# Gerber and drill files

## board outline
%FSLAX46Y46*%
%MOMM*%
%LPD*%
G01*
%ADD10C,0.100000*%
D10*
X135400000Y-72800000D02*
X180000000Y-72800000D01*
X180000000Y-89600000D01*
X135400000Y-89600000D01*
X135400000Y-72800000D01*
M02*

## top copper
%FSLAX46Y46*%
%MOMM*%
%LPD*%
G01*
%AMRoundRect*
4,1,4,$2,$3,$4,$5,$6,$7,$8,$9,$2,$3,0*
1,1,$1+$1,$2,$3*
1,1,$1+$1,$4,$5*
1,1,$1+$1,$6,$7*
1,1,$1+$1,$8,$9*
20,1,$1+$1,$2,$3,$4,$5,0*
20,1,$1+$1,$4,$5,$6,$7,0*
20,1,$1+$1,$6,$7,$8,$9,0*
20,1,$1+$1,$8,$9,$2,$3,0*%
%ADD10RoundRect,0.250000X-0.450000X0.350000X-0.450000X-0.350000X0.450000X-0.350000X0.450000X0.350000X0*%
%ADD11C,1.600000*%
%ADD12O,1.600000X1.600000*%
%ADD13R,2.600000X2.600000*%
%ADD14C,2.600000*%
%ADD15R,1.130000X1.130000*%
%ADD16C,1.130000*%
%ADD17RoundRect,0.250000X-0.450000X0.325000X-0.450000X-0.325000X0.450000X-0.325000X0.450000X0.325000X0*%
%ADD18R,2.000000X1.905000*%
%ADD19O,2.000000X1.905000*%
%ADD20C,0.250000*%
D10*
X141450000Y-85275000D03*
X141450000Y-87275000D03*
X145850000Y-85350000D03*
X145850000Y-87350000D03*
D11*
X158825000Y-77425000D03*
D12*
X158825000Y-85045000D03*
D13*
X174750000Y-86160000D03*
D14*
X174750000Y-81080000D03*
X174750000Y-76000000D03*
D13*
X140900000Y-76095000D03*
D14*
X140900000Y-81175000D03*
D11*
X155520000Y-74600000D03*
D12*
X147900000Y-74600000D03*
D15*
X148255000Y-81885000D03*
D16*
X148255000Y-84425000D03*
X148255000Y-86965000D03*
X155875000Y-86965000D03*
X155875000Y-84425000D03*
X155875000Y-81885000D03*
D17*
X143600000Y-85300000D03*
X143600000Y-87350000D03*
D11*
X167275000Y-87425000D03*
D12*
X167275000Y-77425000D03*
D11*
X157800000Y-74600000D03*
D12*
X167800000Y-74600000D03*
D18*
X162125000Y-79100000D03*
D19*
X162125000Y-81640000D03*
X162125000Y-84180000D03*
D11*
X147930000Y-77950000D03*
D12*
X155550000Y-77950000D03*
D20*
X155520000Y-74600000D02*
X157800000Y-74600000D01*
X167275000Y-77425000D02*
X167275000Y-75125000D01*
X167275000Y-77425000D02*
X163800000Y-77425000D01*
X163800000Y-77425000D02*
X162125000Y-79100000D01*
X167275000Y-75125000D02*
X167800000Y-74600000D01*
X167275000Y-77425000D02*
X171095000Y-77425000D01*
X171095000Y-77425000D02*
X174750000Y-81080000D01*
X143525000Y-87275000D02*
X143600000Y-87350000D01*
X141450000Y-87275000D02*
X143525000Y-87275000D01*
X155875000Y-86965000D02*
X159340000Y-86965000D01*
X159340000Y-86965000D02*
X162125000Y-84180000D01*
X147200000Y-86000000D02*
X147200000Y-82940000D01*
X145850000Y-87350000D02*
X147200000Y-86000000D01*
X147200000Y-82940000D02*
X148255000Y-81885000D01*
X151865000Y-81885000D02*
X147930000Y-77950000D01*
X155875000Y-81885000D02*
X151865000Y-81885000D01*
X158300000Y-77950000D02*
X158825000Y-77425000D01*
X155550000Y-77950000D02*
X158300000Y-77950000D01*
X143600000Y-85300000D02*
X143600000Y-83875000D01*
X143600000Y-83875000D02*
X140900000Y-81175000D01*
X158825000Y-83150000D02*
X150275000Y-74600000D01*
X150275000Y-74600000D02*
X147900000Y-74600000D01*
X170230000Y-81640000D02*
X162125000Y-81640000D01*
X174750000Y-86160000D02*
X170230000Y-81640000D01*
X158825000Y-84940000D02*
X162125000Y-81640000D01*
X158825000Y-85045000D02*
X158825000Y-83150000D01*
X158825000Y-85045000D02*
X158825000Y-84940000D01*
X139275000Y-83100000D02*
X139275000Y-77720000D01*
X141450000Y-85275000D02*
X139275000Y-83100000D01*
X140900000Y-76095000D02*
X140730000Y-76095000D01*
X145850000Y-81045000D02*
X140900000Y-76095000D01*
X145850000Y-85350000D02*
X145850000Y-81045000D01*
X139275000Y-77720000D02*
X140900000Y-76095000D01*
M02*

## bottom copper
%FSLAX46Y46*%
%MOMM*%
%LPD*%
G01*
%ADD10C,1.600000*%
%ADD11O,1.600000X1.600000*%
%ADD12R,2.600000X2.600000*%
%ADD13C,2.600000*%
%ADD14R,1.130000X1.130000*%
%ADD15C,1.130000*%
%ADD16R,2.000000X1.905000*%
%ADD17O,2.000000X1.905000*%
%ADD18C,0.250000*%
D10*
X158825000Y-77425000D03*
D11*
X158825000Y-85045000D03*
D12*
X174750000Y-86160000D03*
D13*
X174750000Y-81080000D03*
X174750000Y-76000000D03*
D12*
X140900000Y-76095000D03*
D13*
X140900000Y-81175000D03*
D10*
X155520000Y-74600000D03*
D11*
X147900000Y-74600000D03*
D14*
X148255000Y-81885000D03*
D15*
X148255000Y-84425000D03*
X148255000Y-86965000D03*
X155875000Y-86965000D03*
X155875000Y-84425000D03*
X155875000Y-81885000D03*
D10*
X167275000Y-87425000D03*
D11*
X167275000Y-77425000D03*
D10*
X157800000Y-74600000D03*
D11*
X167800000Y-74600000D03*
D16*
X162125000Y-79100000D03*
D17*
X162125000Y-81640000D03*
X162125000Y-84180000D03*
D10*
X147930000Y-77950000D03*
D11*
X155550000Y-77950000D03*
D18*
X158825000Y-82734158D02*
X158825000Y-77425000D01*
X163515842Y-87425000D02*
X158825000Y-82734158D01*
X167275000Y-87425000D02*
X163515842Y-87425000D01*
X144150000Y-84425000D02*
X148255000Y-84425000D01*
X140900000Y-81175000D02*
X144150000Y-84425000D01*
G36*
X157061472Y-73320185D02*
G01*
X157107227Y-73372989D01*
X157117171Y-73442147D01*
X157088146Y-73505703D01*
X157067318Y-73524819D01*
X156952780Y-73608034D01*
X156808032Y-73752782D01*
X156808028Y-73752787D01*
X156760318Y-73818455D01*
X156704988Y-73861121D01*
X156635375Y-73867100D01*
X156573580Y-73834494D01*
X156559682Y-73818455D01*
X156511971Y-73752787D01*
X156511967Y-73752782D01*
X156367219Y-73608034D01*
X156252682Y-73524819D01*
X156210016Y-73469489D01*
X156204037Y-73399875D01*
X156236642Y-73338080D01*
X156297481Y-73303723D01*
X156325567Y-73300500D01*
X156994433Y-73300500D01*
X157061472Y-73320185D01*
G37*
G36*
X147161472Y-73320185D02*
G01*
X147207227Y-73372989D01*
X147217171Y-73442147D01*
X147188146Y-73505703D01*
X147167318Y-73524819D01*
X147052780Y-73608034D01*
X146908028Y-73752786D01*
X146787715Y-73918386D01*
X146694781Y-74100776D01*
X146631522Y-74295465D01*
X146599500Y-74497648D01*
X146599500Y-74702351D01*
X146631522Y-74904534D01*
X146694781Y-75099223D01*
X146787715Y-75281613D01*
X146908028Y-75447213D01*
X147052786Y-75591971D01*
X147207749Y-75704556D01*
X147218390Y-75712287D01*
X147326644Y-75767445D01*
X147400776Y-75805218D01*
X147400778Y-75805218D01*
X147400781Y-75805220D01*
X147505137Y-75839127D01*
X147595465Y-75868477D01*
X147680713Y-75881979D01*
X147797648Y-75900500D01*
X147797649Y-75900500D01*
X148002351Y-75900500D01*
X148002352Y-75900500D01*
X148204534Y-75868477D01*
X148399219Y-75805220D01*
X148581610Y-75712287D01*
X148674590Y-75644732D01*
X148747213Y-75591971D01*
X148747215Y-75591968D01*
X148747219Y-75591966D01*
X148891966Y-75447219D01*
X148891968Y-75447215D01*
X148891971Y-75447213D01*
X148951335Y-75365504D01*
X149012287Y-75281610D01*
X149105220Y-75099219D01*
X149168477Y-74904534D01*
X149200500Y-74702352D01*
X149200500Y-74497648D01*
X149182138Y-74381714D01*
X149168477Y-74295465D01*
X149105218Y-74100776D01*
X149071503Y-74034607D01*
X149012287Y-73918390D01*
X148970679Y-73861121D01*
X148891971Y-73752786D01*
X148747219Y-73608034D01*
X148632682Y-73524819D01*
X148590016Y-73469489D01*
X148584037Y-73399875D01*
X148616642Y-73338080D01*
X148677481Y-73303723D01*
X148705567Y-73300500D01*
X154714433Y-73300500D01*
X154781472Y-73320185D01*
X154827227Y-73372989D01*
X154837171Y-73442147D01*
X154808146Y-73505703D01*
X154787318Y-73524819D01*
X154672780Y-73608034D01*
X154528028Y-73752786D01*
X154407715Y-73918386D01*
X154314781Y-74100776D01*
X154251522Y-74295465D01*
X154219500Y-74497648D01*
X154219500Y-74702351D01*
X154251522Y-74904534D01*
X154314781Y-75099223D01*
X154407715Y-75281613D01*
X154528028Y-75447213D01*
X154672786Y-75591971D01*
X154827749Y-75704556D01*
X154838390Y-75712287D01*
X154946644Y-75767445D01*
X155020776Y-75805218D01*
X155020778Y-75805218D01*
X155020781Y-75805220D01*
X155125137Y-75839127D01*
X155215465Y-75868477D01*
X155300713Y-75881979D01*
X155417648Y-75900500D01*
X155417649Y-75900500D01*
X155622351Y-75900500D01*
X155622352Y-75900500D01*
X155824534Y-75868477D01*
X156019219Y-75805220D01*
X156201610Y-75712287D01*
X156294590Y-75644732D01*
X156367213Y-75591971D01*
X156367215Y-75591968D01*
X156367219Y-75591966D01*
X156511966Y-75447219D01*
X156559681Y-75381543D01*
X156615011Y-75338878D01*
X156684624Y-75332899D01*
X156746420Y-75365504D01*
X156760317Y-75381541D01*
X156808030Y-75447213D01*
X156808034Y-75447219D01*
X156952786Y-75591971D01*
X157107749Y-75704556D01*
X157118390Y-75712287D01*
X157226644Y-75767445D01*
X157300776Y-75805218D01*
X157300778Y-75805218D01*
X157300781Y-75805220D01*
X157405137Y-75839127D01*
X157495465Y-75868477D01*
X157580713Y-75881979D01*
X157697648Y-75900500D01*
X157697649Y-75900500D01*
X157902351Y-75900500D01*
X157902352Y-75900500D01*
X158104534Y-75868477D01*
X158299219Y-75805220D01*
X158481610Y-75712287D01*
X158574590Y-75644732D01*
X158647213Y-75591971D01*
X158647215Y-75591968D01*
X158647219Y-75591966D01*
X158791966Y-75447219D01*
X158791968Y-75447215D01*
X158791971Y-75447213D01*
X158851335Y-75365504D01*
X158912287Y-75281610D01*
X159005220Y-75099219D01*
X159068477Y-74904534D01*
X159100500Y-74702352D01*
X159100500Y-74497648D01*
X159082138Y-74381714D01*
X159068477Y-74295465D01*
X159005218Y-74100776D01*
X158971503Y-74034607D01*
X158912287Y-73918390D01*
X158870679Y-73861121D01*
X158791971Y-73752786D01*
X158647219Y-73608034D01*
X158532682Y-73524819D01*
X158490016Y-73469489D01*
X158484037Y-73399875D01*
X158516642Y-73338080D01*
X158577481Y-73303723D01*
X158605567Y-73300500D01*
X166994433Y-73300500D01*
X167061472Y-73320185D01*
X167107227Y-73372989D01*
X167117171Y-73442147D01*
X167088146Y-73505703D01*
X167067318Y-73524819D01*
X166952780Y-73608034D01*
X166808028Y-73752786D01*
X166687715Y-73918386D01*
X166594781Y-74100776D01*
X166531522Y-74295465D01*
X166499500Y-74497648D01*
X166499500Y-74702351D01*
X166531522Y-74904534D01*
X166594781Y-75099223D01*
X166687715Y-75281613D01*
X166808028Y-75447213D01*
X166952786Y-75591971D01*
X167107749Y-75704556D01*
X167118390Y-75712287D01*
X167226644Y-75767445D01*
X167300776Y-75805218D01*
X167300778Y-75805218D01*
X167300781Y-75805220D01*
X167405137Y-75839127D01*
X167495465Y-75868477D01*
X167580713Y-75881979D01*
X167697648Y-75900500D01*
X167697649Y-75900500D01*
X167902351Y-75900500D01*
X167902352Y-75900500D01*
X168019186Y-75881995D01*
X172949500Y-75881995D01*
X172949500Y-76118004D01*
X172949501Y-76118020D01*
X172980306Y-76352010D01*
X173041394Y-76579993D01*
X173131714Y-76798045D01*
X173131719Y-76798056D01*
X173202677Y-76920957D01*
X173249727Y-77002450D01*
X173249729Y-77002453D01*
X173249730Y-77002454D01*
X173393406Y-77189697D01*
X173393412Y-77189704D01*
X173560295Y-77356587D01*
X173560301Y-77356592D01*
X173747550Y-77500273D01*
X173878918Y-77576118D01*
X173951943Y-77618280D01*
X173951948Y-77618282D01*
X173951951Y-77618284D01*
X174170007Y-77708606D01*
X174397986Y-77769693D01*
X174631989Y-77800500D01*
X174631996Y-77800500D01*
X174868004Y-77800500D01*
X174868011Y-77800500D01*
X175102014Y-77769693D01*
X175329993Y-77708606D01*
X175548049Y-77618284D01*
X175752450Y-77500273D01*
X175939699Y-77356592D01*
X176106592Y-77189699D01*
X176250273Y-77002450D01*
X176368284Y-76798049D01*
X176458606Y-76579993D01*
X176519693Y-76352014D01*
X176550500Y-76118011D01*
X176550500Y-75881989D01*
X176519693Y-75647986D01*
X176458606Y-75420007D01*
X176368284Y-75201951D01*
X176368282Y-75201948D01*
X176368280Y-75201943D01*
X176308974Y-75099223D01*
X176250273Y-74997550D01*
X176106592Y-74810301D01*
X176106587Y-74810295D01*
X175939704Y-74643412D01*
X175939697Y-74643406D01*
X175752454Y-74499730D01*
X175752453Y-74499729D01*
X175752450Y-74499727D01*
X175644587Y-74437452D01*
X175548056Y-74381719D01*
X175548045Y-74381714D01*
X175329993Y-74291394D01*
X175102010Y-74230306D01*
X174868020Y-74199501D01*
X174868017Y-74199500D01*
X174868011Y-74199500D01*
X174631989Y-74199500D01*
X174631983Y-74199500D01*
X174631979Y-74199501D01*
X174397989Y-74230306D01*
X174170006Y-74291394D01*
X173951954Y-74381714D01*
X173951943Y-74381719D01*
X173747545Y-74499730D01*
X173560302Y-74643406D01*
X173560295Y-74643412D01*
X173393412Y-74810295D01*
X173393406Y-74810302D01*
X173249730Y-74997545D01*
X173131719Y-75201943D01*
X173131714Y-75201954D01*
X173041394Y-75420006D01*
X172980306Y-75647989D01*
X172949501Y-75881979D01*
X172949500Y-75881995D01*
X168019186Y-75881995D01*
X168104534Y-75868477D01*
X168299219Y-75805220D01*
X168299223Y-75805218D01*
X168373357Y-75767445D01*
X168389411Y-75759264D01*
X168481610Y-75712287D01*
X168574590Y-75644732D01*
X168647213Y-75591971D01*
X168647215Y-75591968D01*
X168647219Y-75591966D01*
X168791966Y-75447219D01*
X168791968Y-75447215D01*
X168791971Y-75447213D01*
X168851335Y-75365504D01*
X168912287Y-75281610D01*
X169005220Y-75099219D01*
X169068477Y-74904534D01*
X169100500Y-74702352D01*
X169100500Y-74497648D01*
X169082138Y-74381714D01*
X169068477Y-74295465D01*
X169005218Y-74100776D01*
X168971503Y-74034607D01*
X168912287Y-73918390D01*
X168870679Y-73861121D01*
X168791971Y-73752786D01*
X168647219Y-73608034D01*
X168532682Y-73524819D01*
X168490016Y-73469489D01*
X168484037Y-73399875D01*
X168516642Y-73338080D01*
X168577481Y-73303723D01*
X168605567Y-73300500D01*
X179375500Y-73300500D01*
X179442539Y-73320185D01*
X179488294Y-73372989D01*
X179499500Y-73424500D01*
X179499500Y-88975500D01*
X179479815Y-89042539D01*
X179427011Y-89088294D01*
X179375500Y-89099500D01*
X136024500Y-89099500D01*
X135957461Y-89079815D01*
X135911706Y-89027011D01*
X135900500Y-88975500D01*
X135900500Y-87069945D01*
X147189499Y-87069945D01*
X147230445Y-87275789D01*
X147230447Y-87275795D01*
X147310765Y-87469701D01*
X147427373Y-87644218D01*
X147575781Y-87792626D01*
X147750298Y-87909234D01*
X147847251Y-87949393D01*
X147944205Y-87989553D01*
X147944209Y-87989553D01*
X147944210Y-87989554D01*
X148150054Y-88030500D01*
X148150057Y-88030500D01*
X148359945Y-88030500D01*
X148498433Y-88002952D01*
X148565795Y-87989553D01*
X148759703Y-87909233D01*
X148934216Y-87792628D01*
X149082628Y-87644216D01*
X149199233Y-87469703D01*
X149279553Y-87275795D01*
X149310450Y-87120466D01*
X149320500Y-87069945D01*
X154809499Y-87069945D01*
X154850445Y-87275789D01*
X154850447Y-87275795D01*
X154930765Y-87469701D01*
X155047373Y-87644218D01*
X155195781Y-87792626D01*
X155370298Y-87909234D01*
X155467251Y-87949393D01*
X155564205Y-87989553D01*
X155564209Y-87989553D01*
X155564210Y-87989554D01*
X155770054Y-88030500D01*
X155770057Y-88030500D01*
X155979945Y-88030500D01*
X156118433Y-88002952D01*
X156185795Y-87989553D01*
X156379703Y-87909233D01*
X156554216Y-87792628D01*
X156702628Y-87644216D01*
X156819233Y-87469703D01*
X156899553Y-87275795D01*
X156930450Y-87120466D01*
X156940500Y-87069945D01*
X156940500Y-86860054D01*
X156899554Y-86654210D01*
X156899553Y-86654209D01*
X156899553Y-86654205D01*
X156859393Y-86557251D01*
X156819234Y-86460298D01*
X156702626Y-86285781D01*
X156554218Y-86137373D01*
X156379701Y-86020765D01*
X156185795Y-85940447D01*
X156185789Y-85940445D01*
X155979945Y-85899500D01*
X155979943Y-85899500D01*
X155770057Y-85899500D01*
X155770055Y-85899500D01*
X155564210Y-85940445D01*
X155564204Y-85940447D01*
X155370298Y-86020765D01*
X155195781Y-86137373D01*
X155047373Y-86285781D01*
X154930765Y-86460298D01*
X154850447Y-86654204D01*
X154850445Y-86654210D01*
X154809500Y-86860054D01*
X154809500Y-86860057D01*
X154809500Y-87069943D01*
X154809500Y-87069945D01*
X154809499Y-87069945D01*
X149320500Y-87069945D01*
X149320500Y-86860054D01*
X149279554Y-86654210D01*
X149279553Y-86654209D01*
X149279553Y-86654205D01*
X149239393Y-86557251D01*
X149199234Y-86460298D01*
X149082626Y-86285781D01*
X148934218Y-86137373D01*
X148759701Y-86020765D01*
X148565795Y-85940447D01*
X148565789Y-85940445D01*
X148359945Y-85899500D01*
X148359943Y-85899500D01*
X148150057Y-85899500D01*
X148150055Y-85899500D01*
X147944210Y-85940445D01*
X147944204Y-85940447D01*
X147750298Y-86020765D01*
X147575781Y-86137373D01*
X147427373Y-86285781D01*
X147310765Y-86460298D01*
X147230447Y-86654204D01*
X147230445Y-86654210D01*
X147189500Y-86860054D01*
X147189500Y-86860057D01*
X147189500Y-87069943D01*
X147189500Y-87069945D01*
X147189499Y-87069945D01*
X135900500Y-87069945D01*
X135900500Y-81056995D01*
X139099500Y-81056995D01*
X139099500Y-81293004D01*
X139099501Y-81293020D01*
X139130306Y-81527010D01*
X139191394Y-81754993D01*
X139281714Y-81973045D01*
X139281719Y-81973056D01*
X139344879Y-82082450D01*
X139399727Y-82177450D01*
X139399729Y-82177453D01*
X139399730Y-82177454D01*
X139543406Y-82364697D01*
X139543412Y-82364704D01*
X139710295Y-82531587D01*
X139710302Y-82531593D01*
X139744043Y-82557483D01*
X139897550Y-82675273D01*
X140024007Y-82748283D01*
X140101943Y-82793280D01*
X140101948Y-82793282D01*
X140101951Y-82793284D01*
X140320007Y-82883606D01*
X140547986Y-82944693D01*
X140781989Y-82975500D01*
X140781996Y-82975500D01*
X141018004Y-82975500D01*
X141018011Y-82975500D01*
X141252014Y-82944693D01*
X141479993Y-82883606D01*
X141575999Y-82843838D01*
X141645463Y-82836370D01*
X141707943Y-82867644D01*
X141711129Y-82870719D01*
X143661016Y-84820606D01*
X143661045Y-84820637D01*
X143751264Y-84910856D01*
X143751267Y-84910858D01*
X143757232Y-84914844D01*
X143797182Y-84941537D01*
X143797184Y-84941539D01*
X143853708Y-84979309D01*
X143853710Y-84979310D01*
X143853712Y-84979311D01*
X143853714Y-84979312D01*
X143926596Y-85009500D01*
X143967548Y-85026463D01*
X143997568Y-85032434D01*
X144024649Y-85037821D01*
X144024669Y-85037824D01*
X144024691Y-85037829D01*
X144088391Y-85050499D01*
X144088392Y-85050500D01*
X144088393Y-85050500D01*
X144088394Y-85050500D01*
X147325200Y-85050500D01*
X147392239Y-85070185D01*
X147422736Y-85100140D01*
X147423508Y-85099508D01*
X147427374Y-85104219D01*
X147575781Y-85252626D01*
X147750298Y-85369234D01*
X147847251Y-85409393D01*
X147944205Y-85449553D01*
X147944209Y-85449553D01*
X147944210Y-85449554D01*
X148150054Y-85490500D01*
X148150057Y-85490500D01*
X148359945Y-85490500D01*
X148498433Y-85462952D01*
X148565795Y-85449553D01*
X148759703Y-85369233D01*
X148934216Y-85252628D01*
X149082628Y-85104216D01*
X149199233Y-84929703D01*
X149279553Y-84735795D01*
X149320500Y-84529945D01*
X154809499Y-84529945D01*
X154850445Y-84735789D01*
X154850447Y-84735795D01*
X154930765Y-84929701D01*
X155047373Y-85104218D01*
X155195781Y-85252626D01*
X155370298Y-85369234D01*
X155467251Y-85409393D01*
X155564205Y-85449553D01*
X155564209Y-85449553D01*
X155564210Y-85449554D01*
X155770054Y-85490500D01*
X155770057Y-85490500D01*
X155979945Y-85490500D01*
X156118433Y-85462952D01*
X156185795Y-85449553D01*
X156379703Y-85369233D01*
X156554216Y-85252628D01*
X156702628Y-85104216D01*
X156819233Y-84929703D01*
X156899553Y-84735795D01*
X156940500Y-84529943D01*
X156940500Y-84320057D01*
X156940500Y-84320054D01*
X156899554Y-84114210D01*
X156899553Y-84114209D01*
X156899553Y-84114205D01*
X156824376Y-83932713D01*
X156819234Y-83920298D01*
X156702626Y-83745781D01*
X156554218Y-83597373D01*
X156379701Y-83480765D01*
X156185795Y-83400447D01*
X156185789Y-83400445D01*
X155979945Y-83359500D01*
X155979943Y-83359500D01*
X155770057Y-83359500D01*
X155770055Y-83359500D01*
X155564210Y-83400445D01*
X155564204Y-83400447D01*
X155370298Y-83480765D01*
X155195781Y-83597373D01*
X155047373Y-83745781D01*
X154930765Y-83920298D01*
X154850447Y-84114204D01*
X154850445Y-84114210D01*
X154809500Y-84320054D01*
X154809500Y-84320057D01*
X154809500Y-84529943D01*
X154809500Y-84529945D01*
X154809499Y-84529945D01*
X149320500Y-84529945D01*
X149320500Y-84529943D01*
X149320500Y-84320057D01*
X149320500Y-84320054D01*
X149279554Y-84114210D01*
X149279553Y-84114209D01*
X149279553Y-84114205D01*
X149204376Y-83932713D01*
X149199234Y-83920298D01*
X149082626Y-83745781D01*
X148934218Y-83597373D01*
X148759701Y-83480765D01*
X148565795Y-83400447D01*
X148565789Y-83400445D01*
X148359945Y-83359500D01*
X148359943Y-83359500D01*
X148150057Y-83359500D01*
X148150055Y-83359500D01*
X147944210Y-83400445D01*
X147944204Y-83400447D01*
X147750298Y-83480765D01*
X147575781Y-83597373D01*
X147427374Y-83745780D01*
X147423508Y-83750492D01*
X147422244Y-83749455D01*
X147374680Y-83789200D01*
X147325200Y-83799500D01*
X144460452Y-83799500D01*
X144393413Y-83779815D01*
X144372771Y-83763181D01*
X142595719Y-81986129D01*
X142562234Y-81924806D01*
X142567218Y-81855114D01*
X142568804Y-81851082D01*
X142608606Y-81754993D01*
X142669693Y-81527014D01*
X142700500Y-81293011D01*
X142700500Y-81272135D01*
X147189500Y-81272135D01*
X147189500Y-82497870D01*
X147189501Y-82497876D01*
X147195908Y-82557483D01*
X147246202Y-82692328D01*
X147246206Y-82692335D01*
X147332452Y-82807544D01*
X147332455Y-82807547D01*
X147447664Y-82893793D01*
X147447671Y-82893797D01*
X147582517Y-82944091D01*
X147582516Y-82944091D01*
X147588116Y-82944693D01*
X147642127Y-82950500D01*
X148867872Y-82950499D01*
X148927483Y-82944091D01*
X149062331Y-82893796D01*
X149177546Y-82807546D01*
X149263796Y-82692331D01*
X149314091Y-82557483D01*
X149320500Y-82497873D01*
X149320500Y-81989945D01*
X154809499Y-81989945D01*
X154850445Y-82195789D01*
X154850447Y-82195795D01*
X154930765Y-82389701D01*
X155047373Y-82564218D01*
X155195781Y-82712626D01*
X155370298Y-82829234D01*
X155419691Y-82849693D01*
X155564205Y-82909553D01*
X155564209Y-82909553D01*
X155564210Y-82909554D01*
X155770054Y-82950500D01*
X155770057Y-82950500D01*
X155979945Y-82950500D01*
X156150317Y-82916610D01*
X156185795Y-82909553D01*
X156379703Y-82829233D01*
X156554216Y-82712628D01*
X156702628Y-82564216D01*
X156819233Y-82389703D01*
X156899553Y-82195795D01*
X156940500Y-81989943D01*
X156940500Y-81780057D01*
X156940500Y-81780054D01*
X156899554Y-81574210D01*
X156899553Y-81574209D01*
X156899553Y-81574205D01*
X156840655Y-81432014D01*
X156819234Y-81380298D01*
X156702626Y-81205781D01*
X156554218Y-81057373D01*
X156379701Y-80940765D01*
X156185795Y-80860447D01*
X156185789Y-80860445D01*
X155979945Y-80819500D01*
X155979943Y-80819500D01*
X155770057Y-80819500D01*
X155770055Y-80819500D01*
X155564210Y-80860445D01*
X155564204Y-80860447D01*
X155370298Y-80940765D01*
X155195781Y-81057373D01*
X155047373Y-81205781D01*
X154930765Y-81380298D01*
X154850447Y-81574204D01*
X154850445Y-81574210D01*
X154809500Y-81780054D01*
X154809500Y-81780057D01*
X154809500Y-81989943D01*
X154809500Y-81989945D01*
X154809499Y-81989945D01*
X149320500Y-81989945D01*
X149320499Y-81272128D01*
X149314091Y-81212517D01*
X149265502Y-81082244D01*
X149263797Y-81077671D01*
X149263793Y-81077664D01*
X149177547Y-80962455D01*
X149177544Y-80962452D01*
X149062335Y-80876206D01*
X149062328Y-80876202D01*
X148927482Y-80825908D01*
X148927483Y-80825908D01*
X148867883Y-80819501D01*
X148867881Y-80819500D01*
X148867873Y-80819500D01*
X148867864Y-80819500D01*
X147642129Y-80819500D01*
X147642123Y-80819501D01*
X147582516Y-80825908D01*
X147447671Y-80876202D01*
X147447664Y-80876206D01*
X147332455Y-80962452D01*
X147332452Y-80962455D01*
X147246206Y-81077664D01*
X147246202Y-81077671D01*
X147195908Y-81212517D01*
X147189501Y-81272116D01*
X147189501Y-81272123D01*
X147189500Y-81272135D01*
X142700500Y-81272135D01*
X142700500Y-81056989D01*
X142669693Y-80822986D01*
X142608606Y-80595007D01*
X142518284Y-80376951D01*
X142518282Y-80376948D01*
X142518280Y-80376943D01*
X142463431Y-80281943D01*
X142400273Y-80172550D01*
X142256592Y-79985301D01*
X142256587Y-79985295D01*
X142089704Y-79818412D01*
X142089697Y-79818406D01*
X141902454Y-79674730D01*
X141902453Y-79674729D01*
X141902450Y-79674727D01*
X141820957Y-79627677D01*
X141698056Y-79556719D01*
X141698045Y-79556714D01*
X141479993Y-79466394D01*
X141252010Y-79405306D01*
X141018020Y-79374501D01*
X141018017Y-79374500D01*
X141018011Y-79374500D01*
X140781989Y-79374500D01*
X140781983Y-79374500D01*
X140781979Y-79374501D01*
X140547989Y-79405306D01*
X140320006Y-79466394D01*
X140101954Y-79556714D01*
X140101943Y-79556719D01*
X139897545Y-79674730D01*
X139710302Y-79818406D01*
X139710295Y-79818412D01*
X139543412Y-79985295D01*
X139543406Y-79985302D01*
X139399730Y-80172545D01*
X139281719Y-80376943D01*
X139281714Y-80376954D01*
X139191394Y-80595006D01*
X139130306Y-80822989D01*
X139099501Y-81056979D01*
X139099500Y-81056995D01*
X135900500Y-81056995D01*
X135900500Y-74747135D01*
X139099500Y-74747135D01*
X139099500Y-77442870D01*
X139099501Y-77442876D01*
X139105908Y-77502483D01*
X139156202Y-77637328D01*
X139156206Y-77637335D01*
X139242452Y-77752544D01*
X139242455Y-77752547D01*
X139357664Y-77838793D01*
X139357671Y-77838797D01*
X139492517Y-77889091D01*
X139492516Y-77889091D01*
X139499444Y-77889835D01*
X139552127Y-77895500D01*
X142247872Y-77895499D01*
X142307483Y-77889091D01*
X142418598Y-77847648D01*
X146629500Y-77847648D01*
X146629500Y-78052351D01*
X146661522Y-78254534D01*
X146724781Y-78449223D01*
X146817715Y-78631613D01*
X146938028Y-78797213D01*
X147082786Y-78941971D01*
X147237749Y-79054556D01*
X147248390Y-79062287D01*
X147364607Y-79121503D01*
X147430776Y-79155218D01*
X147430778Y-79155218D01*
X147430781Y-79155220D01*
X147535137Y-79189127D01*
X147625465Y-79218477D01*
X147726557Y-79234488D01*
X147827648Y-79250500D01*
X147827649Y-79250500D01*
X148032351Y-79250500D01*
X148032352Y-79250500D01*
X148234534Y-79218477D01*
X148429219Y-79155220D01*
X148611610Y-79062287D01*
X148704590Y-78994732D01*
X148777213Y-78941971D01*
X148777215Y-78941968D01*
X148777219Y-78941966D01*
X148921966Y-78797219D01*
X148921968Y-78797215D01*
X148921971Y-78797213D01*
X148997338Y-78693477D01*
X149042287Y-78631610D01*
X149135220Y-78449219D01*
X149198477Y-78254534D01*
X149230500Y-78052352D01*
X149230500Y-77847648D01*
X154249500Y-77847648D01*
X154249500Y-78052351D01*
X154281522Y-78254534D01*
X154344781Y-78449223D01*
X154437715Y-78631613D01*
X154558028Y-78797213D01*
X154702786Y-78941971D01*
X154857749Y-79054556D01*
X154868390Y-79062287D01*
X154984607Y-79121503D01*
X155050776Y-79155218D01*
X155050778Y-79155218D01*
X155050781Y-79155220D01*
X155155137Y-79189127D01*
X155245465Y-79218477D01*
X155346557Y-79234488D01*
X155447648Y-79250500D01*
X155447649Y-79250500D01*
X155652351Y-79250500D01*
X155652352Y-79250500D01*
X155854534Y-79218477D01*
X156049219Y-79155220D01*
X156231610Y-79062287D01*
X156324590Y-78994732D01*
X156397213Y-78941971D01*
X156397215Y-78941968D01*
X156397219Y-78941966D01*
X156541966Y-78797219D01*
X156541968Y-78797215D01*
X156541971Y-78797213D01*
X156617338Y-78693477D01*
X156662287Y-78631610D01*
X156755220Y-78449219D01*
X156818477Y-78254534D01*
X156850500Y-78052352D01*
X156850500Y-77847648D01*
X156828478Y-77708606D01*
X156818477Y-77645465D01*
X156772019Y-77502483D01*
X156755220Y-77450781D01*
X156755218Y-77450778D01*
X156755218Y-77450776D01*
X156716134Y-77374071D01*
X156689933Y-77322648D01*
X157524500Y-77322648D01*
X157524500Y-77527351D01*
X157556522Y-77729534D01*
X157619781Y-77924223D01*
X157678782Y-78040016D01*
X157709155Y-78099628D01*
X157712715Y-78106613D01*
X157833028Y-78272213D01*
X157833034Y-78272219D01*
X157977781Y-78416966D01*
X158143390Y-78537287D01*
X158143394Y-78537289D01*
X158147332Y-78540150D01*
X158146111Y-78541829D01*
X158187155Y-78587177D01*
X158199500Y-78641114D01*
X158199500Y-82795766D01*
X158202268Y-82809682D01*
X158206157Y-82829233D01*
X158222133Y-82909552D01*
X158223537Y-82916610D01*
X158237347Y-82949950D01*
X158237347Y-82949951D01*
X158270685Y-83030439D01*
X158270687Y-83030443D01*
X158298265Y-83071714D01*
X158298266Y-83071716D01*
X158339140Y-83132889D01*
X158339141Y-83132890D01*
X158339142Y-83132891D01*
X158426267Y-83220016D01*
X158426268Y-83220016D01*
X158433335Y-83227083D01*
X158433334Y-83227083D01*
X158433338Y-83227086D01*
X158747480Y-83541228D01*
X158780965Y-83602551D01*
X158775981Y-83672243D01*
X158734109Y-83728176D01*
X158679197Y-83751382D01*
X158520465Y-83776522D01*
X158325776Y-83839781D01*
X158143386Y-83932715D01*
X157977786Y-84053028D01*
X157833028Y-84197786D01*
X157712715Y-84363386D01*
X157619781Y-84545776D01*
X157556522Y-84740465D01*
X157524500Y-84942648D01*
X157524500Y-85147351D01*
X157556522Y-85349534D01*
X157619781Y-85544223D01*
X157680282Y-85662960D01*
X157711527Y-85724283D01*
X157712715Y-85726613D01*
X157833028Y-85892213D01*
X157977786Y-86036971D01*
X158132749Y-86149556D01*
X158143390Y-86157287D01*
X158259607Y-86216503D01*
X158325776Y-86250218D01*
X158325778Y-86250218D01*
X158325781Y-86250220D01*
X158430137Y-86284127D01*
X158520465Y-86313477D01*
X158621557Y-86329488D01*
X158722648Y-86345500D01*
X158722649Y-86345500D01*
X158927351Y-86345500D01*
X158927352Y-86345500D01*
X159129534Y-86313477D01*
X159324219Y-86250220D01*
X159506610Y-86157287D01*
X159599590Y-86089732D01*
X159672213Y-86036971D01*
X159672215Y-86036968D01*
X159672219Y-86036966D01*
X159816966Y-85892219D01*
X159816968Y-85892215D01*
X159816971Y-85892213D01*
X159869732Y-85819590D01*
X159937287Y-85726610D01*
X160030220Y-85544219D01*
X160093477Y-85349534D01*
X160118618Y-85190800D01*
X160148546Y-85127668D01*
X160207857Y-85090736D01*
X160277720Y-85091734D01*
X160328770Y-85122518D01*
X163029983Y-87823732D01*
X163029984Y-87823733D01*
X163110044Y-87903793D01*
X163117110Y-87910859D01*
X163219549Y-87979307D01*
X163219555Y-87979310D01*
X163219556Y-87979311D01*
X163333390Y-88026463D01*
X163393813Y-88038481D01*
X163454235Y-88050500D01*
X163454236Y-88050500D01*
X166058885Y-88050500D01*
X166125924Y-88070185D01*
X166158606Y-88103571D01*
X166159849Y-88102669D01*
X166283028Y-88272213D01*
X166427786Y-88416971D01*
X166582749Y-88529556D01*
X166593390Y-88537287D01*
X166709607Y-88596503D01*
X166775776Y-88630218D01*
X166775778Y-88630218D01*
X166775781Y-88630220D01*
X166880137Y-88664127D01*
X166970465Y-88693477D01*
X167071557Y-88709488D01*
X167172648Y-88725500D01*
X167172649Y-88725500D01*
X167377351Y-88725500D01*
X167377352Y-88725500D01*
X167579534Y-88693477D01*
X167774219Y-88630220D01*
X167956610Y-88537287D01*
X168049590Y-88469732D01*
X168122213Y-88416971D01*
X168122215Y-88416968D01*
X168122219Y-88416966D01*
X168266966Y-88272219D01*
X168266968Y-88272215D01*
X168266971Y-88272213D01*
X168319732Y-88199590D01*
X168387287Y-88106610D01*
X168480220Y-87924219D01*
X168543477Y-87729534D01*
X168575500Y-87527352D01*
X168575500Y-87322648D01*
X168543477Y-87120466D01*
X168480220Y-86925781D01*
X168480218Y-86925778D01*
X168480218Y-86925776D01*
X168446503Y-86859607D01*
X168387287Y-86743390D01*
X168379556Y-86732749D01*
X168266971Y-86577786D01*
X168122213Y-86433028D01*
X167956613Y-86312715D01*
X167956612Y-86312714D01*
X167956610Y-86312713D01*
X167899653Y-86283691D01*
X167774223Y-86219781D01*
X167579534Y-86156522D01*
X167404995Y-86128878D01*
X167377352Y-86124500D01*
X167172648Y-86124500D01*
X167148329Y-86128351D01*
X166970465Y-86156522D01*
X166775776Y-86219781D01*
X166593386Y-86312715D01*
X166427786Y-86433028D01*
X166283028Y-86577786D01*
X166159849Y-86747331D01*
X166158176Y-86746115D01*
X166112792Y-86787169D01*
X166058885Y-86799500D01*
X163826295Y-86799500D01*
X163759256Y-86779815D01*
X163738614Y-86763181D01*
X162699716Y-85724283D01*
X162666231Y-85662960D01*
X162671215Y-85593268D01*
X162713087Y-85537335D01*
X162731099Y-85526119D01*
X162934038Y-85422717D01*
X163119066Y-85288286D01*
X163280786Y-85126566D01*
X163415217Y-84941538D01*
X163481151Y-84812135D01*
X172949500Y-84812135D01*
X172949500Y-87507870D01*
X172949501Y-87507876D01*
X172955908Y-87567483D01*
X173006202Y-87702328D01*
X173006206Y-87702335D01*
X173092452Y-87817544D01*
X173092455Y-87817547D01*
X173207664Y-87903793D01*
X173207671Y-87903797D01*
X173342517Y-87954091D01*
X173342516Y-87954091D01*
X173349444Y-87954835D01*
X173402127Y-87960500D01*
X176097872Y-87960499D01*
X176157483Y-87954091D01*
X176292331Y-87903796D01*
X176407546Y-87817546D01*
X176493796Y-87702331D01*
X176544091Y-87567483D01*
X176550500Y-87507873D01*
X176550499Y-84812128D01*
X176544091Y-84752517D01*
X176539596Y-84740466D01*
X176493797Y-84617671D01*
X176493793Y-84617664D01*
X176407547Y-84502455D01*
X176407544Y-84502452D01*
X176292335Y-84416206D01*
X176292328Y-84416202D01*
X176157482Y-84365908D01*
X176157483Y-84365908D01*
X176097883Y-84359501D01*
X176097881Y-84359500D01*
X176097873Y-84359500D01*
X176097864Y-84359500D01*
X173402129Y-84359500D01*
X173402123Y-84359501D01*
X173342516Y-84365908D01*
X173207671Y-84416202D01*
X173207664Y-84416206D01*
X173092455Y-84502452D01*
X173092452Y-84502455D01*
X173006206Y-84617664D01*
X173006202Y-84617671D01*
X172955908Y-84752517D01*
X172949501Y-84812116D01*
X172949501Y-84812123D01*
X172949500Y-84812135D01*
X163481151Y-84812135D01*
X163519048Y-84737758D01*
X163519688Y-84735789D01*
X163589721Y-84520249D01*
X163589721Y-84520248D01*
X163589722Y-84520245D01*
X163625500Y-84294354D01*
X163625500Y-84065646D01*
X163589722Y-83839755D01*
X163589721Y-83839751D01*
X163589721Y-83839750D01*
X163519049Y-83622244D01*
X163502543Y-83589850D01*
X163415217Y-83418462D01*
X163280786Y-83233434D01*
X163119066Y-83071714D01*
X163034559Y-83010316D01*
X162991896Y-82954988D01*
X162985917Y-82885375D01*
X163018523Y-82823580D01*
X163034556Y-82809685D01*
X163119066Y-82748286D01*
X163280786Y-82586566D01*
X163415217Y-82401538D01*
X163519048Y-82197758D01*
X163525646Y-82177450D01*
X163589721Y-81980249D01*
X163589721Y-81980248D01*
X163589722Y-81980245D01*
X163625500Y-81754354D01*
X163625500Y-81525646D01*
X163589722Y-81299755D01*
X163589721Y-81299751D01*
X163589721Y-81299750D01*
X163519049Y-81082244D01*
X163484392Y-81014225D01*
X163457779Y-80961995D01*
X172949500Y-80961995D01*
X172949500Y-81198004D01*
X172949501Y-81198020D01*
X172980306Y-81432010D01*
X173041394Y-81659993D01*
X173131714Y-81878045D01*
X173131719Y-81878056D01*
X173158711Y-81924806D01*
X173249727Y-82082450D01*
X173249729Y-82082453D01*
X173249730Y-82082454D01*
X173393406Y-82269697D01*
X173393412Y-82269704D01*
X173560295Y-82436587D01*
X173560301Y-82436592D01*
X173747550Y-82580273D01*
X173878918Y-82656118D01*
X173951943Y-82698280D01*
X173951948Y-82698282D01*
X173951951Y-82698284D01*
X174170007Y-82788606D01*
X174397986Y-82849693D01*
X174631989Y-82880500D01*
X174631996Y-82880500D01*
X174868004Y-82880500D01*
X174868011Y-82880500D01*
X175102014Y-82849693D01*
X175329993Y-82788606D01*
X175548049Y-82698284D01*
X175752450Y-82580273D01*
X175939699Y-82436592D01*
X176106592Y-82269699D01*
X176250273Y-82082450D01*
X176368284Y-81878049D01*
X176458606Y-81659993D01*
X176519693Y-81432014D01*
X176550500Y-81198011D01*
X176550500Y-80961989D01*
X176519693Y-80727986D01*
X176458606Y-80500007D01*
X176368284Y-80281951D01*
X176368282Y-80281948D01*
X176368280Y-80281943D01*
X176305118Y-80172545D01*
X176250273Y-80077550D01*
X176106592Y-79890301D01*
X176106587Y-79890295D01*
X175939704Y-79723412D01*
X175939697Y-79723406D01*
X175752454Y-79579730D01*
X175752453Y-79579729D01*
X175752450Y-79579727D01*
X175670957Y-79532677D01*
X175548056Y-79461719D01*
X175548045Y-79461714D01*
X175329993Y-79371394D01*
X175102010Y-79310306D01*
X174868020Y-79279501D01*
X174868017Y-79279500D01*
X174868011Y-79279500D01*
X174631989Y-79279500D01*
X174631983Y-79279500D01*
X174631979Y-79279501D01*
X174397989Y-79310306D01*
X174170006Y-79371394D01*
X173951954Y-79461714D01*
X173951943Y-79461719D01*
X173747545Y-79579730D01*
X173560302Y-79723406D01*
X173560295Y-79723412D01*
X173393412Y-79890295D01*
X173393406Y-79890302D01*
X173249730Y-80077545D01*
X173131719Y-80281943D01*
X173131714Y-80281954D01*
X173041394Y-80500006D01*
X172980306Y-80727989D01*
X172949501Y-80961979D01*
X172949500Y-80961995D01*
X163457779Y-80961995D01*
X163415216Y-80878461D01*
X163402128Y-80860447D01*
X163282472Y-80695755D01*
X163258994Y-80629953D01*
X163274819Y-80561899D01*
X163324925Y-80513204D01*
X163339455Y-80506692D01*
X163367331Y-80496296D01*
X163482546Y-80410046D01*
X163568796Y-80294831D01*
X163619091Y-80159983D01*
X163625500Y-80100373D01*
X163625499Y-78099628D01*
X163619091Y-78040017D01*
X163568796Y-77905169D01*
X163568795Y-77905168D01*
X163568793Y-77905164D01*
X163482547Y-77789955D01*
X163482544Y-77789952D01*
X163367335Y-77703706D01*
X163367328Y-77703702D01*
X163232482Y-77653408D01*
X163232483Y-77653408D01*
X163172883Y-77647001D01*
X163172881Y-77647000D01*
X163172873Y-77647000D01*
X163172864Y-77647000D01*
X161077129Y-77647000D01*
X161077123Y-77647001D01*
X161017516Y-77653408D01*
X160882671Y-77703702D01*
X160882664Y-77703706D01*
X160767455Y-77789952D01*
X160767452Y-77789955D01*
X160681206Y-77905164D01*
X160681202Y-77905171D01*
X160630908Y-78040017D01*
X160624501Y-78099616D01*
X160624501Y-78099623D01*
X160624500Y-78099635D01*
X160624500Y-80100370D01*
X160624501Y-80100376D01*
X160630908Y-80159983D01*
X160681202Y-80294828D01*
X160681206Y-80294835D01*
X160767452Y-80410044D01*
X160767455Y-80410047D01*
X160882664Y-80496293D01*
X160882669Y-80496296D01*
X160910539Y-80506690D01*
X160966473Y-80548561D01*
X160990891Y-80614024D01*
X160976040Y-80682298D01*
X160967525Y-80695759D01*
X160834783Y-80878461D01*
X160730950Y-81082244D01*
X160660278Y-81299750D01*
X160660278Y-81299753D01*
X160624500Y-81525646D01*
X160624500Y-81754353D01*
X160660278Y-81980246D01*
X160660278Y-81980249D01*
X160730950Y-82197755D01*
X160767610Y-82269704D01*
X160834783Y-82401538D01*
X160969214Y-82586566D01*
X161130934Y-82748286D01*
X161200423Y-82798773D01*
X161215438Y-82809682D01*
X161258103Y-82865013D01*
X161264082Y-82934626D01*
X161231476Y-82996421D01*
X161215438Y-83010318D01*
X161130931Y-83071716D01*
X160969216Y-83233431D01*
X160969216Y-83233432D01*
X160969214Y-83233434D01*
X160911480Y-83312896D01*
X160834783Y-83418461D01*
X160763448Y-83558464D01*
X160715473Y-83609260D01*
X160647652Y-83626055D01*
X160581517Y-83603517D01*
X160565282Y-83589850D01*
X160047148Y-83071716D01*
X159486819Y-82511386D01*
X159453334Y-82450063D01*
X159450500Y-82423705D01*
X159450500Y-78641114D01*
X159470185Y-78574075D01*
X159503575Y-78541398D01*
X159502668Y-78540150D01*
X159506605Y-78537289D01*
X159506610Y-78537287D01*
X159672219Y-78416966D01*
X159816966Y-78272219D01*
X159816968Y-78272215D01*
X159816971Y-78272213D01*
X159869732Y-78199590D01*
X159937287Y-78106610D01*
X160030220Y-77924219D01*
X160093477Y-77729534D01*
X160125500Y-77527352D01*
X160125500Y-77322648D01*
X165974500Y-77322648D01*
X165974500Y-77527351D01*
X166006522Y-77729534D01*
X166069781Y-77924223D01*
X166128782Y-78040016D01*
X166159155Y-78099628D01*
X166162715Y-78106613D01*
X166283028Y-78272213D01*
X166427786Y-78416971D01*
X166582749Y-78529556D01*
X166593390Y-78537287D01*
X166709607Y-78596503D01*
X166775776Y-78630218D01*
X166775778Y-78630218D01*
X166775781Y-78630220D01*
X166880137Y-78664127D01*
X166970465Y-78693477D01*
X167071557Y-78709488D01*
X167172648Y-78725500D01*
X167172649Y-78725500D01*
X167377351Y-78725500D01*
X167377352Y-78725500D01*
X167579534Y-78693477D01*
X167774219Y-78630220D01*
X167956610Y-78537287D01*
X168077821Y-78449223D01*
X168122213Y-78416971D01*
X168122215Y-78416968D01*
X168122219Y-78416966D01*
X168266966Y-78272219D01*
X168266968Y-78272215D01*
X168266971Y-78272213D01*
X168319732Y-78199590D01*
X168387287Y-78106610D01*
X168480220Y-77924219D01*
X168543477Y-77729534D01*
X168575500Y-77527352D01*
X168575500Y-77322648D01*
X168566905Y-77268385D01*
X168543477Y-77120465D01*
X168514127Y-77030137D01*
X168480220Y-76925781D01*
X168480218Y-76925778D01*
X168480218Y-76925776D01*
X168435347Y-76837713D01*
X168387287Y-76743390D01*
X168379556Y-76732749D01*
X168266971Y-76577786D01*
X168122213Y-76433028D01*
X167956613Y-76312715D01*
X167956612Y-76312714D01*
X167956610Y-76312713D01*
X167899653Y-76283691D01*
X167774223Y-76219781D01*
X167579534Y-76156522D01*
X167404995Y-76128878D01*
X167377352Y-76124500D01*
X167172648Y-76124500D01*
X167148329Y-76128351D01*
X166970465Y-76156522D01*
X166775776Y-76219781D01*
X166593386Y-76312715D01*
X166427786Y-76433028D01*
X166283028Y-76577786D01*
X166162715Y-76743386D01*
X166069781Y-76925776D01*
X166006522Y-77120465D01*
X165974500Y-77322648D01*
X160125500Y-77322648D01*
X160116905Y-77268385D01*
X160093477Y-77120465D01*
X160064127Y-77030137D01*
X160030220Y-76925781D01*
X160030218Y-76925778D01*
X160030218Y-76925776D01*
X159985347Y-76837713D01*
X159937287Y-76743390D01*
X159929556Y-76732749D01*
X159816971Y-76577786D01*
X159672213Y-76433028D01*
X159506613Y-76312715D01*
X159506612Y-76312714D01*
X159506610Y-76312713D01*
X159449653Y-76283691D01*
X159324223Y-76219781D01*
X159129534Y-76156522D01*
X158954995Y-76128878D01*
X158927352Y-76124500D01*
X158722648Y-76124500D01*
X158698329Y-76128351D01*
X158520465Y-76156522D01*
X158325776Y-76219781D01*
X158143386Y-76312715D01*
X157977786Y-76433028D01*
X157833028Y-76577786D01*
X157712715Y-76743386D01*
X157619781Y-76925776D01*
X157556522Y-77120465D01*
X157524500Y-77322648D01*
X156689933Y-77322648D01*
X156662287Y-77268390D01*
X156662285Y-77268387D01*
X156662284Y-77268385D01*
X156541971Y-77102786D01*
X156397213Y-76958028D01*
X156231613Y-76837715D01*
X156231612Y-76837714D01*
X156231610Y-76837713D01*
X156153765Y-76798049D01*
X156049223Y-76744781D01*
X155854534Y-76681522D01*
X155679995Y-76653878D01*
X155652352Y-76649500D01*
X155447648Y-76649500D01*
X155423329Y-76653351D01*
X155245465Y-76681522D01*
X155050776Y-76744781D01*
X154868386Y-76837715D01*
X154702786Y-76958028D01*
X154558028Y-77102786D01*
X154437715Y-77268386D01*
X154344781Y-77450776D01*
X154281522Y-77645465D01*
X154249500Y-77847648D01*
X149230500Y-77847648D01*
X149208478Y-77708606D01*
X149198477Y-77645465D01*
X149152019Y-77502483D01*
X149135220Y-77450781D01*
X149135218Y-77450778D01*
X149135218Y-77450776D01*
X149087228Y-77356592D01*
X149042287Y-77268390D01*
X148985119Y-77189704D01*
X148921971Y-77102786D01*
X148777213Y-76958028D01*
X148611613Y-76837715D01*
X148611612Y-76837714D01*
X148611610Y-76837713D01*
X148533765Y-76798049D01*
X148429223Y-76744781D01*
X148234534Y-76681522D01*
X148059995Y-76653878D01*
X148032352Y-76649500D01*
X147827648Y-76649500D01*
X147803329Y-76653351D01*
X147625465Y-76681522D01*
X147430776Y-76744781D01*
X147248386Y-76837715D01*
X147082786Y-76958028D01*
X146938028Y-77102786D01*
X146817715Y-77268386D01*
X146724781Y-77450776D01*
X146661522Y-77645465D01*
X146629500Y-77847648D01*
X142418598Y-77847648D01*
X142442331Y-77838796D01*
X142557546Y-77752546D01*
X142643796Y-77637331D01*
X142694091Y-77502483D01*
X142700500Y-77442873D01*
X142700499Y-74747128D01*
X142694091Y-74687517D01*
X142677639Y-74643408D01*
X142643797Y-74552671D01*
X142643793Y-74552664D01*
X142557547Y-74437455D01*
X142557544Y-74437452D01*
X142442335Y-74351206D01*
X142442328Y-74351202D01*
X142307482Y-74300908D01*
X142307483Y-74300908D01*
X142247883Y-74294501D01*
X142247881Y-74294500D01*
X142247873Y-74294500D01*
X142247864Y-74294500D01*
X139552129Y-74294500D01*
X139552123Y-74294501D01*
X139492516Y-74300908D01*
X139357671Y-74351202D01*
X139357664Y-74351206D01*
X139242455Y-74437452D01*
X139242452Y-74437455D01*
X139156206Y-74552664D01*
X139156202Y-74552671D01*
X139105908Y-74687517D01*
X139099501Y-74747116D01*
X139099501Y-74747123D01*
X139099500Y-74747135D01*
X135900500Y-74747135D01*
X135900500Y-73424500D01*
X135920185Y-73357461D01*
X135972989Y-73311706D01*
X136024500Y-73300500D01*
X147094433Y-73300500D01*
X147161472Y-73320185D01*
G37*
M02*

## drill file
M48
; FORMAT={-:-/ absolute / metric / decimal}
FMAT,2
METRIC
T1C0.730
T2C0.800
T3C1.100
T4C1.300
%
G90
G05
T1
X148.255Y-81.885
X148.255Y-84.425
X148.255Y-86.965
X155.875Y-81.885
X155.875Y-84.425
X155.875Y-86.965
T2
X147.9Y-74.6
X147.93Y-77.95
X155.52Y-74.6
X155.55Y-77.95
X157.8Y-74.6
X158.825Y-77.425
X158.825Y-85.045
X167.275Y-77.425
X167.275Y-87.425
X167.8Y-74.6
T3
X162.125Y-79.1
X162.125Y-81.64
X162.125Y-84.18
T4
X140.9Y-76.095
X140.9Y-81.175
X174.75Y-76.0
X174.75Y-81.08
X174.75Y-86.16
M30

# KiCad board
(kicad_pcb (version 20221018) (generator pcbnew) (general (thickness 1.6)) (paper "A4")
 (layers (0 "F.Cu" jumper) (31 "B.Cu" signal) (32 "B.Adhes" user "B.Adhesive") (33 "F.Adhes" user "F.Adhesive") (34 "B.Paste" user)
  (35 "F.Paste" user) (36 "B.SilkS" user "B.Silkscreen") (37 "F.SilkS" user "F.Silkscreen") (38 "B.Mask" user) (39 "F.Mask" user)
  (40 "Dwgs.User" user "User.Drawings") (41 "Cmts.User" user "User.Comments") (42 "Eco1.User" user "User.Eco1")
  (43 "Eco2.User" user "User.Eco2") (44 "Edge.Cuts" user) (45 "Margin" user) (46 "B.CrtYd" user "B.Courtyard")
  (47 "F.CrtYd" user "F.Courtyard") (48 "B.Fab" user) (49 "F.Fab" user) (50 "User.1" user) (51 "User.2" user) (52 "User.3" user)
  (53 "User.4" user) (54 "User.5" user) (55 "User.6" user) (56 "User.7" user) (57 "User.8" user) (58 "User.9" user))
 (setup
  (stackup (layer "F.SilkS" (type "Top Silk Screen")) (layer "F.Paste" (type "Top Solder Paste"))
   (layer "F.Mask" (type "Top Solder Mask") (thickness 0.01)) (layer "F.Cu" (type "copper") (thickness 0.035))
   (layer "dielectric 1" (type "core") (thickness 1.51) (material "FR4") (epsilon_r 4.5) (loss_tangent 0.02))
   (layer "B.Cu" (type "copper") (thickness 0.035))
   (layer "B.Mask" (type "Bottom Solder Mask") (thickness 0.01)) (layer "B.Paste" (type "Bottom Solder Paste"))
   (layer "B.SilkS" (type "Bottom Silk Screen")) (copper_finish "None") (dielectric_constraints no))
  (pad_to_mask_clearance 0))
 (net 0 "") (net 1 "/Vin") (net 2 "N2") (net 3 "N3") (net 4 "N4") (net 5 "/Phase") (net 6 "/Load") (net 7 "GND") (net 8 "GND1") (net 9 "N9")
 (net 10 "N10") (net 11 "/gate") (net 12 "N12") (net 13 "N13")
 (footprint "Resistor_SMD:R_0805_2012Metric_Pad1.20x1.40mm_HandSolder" (layer "F.Cu") (at 141.45 86.275 -90)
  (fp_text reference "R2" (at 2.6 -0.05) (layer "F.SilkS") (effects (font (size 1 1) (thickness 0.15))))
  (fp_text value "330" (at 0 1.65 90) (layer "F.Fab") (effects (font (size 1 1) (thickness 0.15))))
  (pad "1" smd roundrect (at -1 0 270) (size 1.2 1.4) (layers "F.Cu" "F.Paste" "F.Mask") (roundrect_rratio 0.208333) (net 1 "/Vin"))
  (pad "2" smd roundrect (at 1 0 270) (size 1.2 1.4) (layers "F.Cu" "F.Paste" "F.Mask") (roundrect_rratio 0.208333) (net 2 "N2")))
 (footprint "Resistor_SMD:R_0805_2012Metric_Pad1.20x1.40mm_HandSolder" (layer "F.Cu") (at 145.85 86.35 -90)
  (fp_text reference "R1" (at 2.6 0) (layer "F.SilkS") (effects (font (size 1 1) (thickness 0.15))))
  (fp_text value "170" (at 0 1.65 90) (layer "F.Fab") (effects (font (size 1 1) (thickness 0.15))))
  (pad "1" smd roundrect (at -1 0 270) (size 1.2 1.4) (layers "F.Cu" "F.Paste" "F.Mask") (roundrect_rratio 0.208333) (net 1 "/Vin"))
  (pad "2" smd roundrect (at 1 0 270) (size 1.2 1.4) (layers "F.Cu" "F.Paste" "F.Mask") (roundrect_rratio 0.208333) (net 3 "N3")))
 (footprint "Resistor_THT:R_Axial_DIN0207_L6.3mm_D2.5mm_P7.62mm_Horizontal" (layer "F.Cu") (at 158.825 77.425 -90)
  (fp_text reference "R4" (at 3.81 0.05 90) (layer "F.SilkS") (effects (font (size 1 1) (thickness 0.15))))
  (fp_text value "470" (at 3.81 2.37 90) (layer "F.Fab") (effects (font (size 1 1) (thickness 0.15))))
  (pad "1" thru_hole circle (at 0 0 270) (size 1.6 1.6) (drill 0.8) (layers "*.Cu" "*.Mask") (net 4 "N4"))
  (pad "2" thru_hole oval (at 7.62 0 270) (size 1.6 1.6) (drill 0.8) (layers "*.Cu" "*.Mask") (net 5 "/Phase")))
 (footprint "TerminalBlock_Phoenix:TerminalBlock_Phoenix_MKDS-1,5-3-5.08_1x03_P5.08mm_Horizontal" (layer "F.Cu") (at 174.75 86.16 90)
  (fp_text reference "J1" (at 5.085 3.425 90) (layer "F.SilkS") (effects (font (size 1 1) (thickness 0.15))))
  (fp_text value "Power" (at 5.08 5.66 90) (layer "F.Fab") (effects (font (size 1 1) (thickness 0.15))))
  (pad "1" thru_hole rect (at 0 0 90) (size 2.6 2.6) (drill 1.3) (layers "*.Cu" "*.Mask") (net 5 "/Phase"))
  (pad "2" thru_hole circle (at 5.08 0 90) (size 2.6 2.6) (drill 1.3) (layers "*.Cu" "*.Mask") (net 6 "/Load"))
  (pad "3" thru_hole circle (at 10.16 0 90) (size 2.6 2.6) (drill 1.3) (layers "*.Cu" "*.Mask") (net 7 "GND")))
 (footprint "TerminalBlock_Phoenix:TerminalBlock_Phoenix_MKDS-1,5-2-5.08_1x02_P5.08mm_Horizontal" (layer "F.Cu") (at 140.9 76.095 -90)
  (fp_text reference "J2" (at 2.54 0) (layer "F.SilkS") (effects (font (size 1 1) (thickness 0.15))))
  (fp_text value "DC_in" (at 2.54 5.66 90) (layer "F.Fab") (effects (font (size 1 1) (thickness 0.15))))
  (pad "1" thru_hole rect (at 0 0 270) (size 2.6 2.6) (drill 1.3) (layers "*.Cu" "*.Mask") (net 1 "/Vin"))
  (pad "2" thru_hole circle (at 5.08 0 270) (size 2.6 2.6) (drill 1.3) (layers "*.Cu" "*.Mask") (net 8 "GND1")))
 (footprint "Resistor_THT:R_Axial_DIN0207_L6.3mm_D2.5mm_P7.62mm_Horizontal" (layer "F.Cu") (at 155.52 74.6 180)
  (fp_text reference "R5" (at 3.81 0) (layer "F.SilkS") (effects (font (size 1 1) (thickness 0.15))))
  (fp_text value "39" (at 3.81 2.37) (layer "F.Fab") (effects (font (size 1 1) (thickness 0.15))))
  (pad "1" thru_hole circle (at 0 0 180) (size 1.6 1.6) (drill 0.8) (layers "*.Cu" "*.Mask") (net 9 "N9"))
  (pad "2" thru_hole oval (at 7.62 0 180) (size 1.6 1.6) (drill 0.8) (layers "*.Cu" "*.Mask") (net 5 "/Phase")))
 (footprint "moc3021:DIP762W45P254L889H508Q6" (layer "F.Cu") (at 152.065 84.425)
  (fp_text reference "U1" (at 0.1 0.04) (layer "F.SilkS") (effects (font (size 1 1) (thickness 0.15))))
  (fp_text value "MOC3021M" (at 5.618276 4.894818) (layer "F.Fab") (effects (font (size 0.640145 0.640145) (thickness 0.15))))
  (pad "1" thru_hole rect (at -3.81 -2.54) (size 1.13 1.13) (drill 0.73) (layers "*.Cu" "*.Mask") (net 3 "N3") (solder_mask_margin 0.102))
  (pad "2" thru_hole circle (at -3.81 0) (size 1.13 1.13) (drill 0.73) (layers "*.Cu" "*.Mask") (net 8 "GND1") (solder_mask_margin 0.102))
  (pad "3" thru_hole circle (at -3.81 2.54) (size 1.13 1.13) (drill 0.73) (layers "*.Cu" "*.Mask") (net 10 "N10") (solder_mask_margin 0.102))
  (pad "4" thru_hole circle (at 3.81 2.54) (size 1.13 1.13) (drill 0.73) (layers "*.Cu" "*.Mask") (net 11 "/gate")
   (solder_mask_margin 0.102))
  (pad "5" thru_hole circle (at 3.81 0) (size 1.13 1.13) (drill 0.73) (layers "*.Cu" "*.Mask") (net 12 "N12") (solder_mask_margin 0.102))
  (pad "6" thru_hole circle (at 3.81 -2.54) (size 1.13 1.13) (drill 0.73) (layers "*.Cu" "*.Mask") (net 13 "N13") (solder_mask_margin 0.102)))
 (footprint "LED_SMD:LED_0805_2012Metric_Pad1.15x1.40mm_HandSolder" (layer "F.Cu") (at 143.6 86.325 -90)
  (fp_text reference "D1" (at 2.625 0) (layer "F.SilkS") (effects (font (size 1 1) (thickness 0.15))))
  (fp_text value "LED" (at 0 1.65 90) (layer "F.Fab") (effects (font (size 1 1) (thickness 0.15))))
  (pad "1" smd roundrect (at -1.025 0 270) (size 1.15 1.4) (layers "F.Cu" "F.Paste" "F.Mask") (roundrect_rratio 0.217391) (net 8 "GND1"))
  (pad "2" smd roundrect (at 1.025 0 270) (size 1.15 1.4) (layers "F.Cu" "F.Paste" "F.Mask") (roundrect_rratio 0.217391) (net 2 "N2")))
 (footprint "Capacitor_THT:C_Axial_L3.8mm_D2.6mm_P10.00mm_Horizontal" (layer "F.Cu") (at 167.275 87.425 90)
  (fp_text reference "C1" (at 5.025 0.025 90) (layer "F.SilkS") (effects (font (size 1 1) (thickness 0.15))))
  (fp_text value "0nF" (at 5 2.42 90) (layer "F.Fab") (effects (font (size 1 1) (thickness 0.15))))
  (pad "1" thru_hole circle (at 0 0 90) (size 1.6 1.6) (drill 0.8) (layers "*.Cu" "*.Mask") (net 4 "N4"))
  (pad "2" thru_hole oval (at 10 0 90) (size 1.6 1.6) (drill 0.8) (layers "*.Cu" "*.Mask") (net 6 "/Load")))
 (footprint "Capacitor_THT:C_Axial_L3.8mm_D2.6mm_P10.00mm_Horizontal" (layer "F.Cu") (at 157.8 74.6)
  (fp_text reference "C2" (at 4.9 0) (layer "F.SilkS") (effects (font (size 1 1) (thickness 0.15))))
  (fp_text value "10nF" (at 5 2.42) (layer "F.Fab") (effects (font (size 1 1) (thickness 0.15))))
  (pad "1" thru_hole circle (at 0 0) (size 1.6 1.6) (drill 0.8) (layers "*.Cu" "*.Mask") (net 9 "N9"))
  (pad "2" thru_hole oval (at 10 0) (size 1.6 1.6) (drill 0.8) (layers "*.Cu" "*.Mask") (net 6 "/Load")))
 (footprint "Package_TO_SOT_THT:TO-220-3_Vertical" (layer "F.Cu") (at 162.125 79.1 -90)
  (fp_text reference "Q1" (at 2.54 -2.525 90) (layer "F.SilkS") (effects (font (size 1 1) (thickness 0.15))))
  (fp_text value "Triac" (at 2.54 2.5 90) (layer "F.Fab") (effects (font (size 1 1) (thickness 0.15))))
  (pad "1" thru_hole rect (at 0 0 270) (size 1.905 2) (drill 1.1) (layers "*.Cu" "*.Mask") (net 6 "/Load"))
  (pad "2" thru_hole oval (at 2.54 0 270) (size 1.905 2) (drill 1.1) (layers "*.Cu" "*.Mask") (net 5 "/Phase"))
  (pad "3" thru_hole oval (at 5.08 0 270) (size 1.905 2) (drill 1.1) (layers "*.Cu" "*.Mask") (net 11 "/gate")))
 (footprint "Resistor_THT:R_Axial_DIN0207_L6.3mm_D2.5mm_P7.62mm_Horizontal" (layer "F.Cu") (at 147.93 77.95)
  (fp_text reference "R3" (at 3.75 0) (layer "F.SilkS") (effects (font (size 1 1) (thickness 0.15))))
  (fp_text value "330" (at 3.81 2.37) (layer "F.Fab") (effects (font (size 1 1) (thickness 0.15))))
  (pad "1" thru_hole circle (at 0 0) (size 1.6 1.6) (drill 0.8) (layers "*.Cu" "*.Mask") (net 13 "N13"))
  (pad "2" thru_hole oval (at 7.62 0) (size 1.6 1.6) (drill 0.8) (layers "*.Cu" "*.Mask") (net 4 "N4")))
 (gr_rect (start 135.4 72.8) (end 180 89.6) (stroke (width 0.1) (type default)) (fill none) (layer "Edge.Cuts"))
 (segment (start 155.52 74.6) (end 157.8 74.6) (width 0.25) (layer "F.Cu") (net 9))
 (segment (start 167.275 77.425) (end 167.275 75.125) (width 0.25) (layer "F.Cu") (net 6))
 (segment (start 167.275 77.425) (end 163.8 77.425) (width 0.25) (layer "F.Cu") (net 6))
 (segment (start 163.8 77.425) (end 162.125 79.1) (width 0.25) (layer "F.Cu") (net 6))
 (segment (start 167.275 75.125) (end 167.8 74.6) (width 0.25) (layer "F.Cu") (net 6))
 (segment (start 167.275 77.425) (end 171.095 77.425) (width 0.25) (layer "F.Cu") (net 6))
 (segment (start 171.095 77.425) (end 174.75 81.08) (width 0.25) (layer "F.Cu") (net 6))
 (segment (start 143.525 87.275) (end 143.6 87.35) (width 0.25) (layer "F.Cu") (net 2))
 (segment (start 141.45 87.275) (end 143.525 87.275) (width 0.25) (layer "F.Cu") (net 2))
 (segment (start 155.875 86.965) (end 159.34 86.965) (width 0.25) (layer "F.Cu") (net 11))
 (segment (start 159.34 86.965) (end 162.125 84.18) (width 0.25) (layer "F.Cu") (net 11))
 (segment (start 147.2 86) (end 147.2 82.94) (width 0.25) (layer "F.Cu") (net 3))
 (segment (start 145.85 87.35) (end 147.2 86) (width 0.25) (layer "F.Cu") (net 3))
 (segment (start 147.2 82.94) (end 148.255 81.885) (width 0.25) (layer "F.Cu") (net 3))
 (segment (start 151.865 81.885) (end 147.93 77.95) (width 0.25) (layer "F.Cu") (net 13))
 (segment (start 155.875 81.885) (end 151.865 81.885) (width 0.25) (layer "F.Cu") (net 13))
 (segment (start 158.3 77.95) (end 158.825 77.425) (width 0.25) (layer "F.Cu") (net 4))
 (segment (start 155.55 77.95) (end 158.3 77.95) (width 0.25) (layer "F.Cu") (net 4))
 (segment (start 158.825 82.734158) (end 158.825 77.425) (width 0.25) (layer "B.Cu") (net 4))
 (segment (start 163.515842 87.425) (end 158.825 82.734158) (width 0.25) (layer "B.Cu") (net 4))
 (segment (start 167.275 87.425) (end 163.515842 87.425) (width 0.25) (layer "B.Cu") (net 4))
 (segment (start 143.6 85.3) (end 143.6 83.875) (width 0.25) (layer "F.Cu") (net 8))
 (segment (start 143.6 83.875) (end 140.9 81.175) (width 0.25) (layer "F.Cu") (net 8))
 (segment (start 144.15 84.425) (end 148.255 84.425) (width 0.25) (layer "B.Cu") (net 8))
 (segment (start 140.9 81.175) (end 144.15 84.425) (width 0.25) (layer "B.Cu") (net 8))
 (segment (start 158.825 83.15) (end 150.275 74.6) (width 0.25) (layer "F.Cu") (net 5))
 (segment (start 150.275 74.6) (end 147.9 74.6) (width 0.25) (layer "F.Cu") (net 5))
 (segment (start 170.23 81.64) (end 162.125 81.64) (width 0.25) (layer "F.Cu") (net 5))
 (segment (start 174.75 86.16) (end 170.23 81.64) (width 0.25) (layer "F.Cu") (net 5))
 (segment (start 158.825 84.94) (end 162.125 81.64) (width 0.25) (layer "F.Cu") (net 5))
 (segment (start 158.825 85.045) (end 158.825 83.15) (width 0.25) (layer "F.Cu") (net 5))
 (segment (start 158.825 85.045) (end 158.825 84.94) (width 0.25) (layer "F.Cu") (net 5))
 (segment (start 139.275 83.1) (end 139.275 77.72) (width 0.25) (layer "F.Cu") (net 1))
 (segment (start 141.45 85.275) (end 139.275 83.1) (width 0.25) (layer "F.Cu") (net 1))
 (segment (start 140.9 76.095) (end 140.73 76.095) (width 0.25) (layer "F.Cu") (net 1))
 (segment (start 145.85 81.045) (end 140.9 76.095) (width 0.25) (layer "F.Cu") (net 1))
 (segment (start 145.85 85.35) (end 145.85 81.045) (width 0.25) (layer "F.Cu") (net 1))
 (segment (start 139.275 77.72) (end 140.9 76.095) (width 0.25) (layer "F.Cu") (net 1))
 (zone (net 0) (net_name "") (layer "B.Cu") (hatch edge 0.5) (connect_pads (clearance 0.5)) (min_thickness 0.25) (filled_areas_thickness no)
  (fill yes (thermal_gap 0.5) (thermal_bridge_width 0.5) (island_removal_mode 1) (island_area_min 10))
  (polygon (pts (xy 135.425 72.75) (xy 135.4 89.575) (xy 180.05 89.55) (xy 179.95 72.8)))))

